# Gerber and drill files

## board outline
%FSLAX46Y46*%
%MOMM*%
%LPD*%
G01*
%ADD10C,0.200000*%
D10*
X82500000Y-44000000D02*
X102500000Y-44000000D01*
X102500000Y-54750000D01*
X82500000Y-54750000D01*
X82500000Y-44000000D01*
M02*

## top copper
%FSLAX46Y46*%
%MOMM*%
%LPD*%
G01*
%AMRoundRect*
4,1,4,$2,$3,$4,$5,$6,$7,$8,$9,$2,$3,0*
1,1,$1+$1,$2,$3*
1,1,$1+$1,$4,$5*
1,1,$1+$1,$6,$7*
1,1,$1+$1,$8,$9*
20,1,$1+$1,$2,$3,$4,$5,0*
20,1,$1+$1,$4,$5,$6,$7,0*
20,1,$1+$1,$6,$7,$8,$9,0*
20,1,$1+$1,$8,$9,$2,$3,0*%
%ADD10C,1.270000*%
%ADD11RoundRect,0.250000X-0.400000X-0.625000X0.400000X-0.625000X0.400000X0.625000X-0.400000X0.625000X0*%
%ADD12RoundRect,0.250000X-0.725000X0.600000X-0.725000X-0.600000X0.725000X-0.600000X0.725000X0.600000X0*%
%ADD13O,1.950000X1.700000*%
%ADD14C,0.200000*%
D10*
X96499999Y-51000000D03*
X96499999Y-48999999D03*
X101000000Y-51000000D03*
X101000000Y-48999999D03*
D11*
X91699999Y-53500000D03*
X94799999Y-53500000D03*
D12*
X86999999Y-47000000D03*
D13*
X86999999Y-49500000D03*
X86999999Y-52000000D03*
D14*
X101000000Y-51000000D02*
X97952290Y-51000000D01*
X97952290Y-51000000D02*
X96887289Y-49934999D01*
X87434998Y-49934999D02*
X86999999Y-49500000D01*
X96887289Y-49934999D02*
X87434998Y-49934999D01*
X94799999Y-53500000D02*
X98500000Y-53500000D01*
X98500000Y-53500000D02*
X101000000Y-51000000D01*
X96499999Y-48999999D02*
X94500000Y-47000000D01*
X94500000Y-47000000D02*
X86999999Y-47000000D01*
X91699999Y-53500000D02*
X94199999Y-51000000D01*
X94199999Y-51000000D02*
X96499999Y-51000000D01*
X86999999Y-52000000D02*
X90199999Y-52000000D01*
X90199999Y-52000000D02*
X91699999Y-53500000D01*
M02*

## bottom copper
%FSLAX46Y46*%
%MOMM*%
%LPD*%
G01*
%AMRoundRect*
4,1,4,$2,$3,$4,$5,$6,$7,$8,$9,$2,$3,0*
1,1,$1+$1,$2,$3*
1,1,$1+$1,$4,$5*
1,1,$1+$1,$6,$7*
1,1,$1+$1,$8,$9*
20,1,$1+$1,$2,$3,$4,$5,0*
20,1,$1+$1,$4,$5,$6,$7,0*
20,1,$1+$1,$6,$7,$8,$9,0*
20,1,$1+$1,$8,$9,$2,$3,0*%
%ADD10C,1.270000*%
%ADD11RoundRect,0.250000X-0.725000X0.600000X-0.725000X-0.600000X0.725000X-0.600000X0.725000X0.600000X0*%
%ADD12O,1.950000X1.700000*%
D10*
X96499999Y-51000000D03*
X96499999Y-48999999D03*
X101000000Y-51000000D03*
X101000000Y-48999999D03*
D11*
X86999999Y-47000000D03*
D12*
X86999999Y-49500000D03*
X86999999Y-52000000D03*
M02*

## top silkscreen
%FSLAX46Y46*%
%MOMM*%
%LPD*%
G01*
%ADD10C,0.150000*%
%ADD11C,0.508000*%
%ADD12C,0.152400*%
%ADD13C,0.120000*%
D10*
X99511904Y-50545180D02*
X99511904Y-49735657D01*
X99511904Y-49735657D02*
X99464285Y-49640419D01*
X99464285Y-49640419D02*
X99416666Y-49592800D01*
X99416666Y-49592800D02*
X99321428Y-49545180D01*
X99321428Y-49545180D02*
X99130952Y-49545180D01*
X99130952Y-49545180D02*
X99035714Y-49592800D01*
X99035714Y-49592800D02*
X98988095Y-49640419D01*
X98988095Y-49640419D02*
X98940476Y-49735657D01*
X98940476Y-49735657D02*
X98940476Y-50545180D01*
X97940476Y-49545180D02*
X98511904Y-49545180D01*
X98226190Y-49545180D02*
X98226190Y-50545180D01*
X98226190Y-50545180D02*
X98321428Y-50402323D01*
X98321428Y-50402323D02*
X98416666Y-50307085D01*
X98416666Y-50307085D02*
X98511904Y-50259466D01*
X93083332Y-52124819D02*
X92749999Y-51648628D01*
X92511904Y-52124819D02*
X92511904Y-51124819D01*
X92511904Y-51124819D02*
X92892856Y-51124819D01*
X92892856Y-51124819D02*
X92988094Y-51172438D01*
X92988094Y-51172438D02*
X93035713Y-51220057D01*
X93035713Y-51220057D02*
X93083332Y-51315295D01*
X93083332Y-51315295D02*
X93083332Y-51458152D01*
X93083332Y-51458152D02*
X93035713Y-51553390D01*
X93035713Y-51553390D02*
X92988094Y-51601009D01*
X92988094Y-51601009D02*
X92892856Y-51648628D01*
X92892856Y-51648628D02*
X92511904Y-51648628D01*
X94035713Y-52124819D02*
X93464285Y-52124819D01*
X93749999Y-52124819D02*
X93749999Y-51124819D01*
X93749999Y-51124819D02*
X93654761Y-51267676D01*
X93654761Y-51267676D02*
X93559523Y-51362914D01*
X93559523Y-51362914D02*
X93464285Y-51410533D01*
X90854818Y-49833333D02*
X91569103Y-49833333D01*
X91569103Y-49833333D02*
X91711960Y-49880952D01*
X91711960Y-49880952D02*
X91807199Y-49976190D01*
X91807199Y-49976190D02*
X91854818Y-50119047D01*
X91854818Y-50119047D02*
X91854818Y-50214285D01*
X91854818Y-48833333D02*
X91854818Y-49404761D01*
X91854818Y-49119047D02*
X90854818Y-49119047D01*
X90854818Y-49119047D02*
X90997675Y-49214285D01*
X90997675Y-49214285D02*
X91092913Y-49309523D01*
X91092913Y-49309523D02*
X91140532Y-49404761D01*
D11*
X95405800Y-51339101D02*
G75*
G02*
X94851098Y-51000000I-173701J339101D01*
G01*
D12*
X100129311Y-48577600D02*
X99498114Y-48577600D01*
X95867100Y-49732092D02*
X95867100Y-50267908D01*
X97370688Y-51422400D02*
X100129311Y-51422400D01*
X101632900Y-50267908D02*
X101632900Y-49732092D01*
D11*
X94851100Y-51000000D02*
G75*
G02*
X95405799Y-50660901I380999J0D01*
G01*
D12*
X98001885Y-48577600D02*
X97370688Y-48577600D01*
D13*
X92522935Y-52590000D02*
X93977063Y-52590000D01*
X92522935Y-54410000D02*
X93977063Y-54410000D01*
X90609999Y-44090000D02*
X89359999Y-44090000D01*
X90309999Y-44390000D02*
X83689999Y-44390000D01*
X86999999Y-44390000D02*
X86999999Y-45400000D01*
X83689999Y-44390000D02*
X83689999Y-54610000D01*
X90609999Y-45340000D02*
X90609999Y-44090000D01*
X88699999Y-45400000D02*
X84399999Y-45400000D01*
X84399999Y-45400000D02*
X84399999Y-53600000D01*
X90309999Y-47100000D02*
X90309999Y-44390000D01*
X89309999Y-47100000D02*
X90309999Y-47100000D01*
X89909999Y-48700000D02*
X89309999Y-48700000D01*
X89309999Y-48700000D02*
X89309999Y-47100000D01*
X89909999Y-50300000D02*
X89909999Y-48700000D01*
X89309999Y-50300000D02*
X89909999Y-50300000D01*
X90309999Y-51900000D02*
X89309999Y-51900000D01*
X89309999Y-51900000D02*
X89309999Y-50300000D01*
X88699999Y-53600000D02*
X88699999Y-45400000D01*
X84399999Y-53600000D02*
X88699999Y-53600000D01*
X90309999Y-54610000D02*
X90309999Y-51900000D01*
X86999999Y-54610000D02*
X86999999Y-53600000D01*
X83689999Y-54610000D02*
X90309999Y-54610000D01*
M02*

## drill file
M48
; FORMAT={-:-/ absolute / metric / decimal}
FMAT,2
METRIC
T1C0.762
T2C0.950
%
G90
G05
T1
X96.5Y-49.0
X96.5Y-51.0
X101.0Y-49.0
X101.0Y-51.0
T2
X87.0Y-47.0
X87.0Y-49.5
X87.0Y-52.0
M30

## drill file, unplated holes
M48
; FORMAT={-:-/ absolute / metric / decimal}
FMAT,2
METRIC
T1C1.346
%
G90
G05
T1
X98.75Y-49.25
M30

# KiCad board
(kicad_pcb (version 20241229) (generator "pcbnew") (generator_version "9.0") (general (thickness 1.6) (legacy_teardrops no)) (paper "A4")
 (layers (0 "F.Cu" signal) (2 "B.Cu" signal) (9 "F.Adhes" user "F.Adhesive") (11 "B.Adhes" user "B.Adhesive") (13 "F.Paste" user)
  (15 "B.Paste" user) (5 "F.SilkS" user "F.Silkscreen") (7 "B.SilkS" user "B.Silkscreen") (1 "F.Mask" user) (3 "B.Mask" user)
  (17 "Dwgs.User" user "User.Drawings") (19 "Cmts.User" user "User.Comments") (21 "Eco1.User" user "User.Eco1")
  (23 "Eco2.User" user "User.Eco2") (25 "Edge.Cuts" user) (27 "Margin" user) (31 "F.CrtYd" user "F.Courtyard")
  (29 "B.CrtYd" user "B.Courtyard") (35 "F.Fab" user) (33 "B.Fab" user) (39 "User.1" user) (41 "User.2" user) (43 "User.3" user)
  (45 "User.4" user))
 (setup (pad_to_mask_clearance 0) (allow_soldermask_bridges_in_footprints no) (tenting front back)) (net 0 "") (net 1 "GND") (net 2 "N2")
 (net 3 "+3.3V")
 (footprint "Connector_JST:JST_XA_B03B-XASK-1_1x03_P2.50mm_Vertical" (layer "F.Cu") (at 86.999999 47 -90)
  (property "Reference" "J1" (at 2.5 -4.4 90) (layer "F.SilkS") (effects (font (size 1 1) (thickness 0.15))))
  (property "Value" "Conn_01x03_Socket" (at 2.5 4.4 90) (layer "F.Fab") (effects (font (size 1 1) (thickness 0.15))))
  (fp_line (start -2.61 3.31) (end 7.61 3.31) (stroke (width 0.12) (type solid)) (layer "F.SilkS"))
  (fp_line (start 7.61 3.31) (end 7.61 -3.31) (stroke (width 0.12) (type solid)) (layer "F.SilkS"))
  (fp_line (start -1.6 2.6) (end 6.6 2.6) (stroke (width 0.12) (type solid)) (layer "F.SilkS"))
  (fp_line (start 6.6 2.6) (end 6.6 -1.7) (stroke (width 0.12) (type solid)) (layer "F.SilkS"))
  (fp_line (start -2.61 0) (end -1.6 0) (stroke (width 0.12) (type solid)) (layer "F.SilkS"))
  (fp_line (start 7.61 0) (end 6.6 0) (stroke (width 0.12) (type solid)) (layer "F.SilkS"))
  (fp_line (start -1.6 -1.7) (end -1.6 2.6) (stroke (width 0.12) (type solid)) (layer "F.SilkS"))
  (fp_line (start 6.6 -1.7) (end -1.6 -1.7) (stroke (width 0.12) (type solid)) (layer "F.SilkS"))
  (fp_line (start 0.1 -2.31) (end 0.1 -3.31) (stroke (width 0.12) (type solid)) (layer "F.SilkS"))
  (fp_line (start 1.7 -2.31) (end 0.1 -2.31) (stroke (width 0.12) (type solid)) (layer "F.SilkS"))
  (fp_line (start 3.3 -2.31) (end 3.3 -2.91) (stroke (width 0.12) (type solid)) (layer "F.SilkS"))
  (fp_line (start 4.9 -2.31) (end 3.3 -2.31) (stroke (width 0.12) (type solid)) (layer "F.SilkS"))
  (fp_line (start 1.7 -2.91) (end 1.7 -2.31) (stroke (width 0.12) (type solid)) (layer "F.SilkS"))
  (fp_line (start 3.3 -2.91) (end 1.7 -2.91) (stroke (width 0.12) (type solid)) (layer "F.SilkS"))
  (fp_line (start -2.61 -3.31) (end -2.61 3.31) (stroke (width 0.12) (type solid)) (layer "F.SilkS"))
  (fp_line (start 0.1 -3.31) (end -2.61 -3.31) (stroke (width 0.12) (type solid)) (layer "F.SilkS"))
  (fp_line (start 4.9 -3.31) (end 4.9 -2.31) (stroke (width 0.12) (type solid)) (layer "F.SilkS"))
  (fp_line (start 7.61 -3.31) (end 4.9 -3.31) (stroke (width 0.12) (type solid)) (layer "F.SilkS"))
  (fp_line (start -2.91 -3.61) (end -2.91 -2.36) (stroke (width 0.12) (type solid)) (layer "F.SilkS"))
  (fp_line (start -1.66 -3.61) (end -2.91 -3.61) (stroke (width 0.12) (type solid)) (layer "F.SilkS"))
  (pad "1" thru_hole roundrect (at 0 0 270) (size 1.7 1.95) (drill 0.95) (layers "*.Cu" "*.Mask") (remove_unused_layers no)
   (roundrect_rratio 0.147059) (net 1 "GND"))
  (pad "2" thru_hole oval (at 2.5 0 270) (size 1.7 1.95) (drill 0.95) (layers "*.Cu" "*.Mask") (remove_unused_layers no) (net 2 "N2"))
  (pad "3" thru_hole oval (at 5 0 270) (size 1.7 1.95) (drill 0.95) (layers "*.Cu" "*.Mask") (remove_unused_layers no) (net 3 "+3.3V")))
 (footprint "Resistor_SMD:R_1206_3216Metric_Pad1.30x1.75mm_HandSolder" (layer "F.Cu") (at 93.249999 53.5)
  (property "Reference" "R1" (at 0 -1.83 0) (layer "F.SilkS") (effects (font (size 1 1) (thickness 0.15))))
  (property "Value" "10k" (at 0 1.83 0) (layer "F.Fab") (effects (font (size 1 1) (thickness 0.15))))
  (fp_line (start -0.727064 -0.91) (end 0.727064 -0.91) (stroke (width 0.12) (type solid)) (layer "F.SilkS"))
  (fp_line (start -0.727064 0.91) (end 0.727064 0.91) (stroke (width 0.12) (type solid)) (layer "F.SilkS"))
  (pad "1" smd roundrect (at -1.55 0) (size 1.3 1.75) (layers "F.Cu" "F.Mask" "F.Paste") (roundrect_rratio 0.192308) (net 3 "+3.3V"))
  (pad "2" smd roundrect (at 1.55 0) (size 1.3 1.75) (layers "F.Cu" "F.Mask" "F.Paste") (roundrect_rratio 0.192308) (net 2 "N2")))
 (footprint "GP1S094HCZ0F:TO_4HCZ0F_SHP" (layer "F.Cu") (at 96.499999 51 180)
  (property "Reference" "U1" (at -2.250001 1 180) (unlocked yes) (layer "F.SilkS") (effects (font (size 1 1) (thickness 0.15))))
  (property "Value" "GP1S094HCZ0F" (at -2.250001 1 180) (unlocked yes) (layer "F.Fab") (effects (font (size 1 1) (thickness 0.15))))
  (fp_line (start 0.632899 1.267908) (end 0.632899 0.732092) (stroke (width 0.1524) (type solid)) (layer "F.SilkS"))
  (fp_line (start -0.870689 -0.4224) (end -3.629312 -0.4224) (stroke (width 0.1524) (type solid)) (layer "F.SilkS"))
  (fp_line (start -1.501886 2.4224) (end -0.870689 2.4224) (stroke (width 0.1524) (type solid)) (layer "F.SilkS"))
  (fp_line (start -3.629312 2.4224) (end -2.998115 2.4224) (stroke (width 0.1524) (type solid)) (layer "F.SilkS"))
  (fp_line (start -5.132901 0.732092) (end -5.132901 1.267908) (stroke (width 0.1524) (type solid)) (layer "F.SilkS"))
  (fp_arc (start 1.648899 0) (mid 1.466622 0.32507) (end 1.094199 0.339101) (stroke (width 0.508) (type solid)) (layer "F.SilkS"))
  (fp_arc (start 1.094199 -0.339101) (mid 1.466622 -0.32507) (end 1.648899 0) (stroke (width 0.508) (type solid)) (layer "F.SilkS"))
  (pad "" np_thru_hole circle (at -2.250001 1.750062 180) (size 1.3462 1.3462) (drill 1.3462) (layers "*.Cu" "*.Mask"))
  (pad "1" thru_hole circle (at 0 0 180) (size 1.27 1.27) (drill 0.762) (layers "*.Cu" "*.Mask") (remove_unused_layers no) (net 3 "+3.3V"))
  (pad "2" thru_hole circle (at -4.500001 0 180) (size 1.27 1.27) (drill 0.762) (layers "*.Cu" "*.Mask") (remove_unused_layers no)
   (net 2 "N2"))
  (pad "3" thru_hole circle (at -4.500001 2.000001 180) (size 1.27 1.27) (drill 0.762) (layers "*.Cu" "*.Mask") (remove_unused_layers no)
   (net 1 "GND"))
  (pad "4" thru_hole circle (at 0 2.000001 180) (size 1.27 1.27) (drill 0.762) (layers "*.Cu" "*.Mask") (remove_unused_layers no)
   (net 1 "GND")))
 (gr_rect (start 82.5 44) (end 102.5 54.75) (stroke (width 0.2) (type solid)) (fill no) (layer "Edge.Cuts"))
 (segment (start 94.799999 53.5) (end 98.5 53.5) (width 0.2) (layer "F.Cu") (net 2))
 (segment (start 101 51) (end 97.95229 51) (width 0.2) (layer "F.Cu") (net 2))
 (segment (start 87.434998 49.934999) (end 86.999999 49.5) (width 0.2) (layer "F.Cu") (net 2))
 (segment (start 96.887289 49.934999) (end 87.434998 49.934999) (width 0.2) (layer "F.Cu") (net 2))
 (segment (start 97.95229 51) (end 96.887289 49.934999) (width 0.2) (layer "F.Cu") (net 2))
 (segment (start 98.5 53.5) (end 101 51) (width 0.2) (layer "F.Cu") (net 2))
 (segment (start 94.199999 51) (end 96.499999 51) (width 0.2) (layer "F.Cu") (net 3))
 (segment (start 90.199999 52) (end 91.699999 53.5) (width 0.2) (layer "F.Cu") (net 3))
 (segment (start 91.699999 53.5) (end 94.199999 51) (width 0.2) (layer "F.Cu") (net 3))
 (segment (start 86.999999 52) (end 90.199999 52) (width 0.2) (layer "F.Cu") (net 3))
 (segment (start 94.5 47) (end 86.999999 47) (width 0.2) (layer "F.Cu") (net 1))
 (segment (start 96.499999 48.999999) (end 94.5 47) (width 0.2) (layer "F.Cu") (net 1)))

